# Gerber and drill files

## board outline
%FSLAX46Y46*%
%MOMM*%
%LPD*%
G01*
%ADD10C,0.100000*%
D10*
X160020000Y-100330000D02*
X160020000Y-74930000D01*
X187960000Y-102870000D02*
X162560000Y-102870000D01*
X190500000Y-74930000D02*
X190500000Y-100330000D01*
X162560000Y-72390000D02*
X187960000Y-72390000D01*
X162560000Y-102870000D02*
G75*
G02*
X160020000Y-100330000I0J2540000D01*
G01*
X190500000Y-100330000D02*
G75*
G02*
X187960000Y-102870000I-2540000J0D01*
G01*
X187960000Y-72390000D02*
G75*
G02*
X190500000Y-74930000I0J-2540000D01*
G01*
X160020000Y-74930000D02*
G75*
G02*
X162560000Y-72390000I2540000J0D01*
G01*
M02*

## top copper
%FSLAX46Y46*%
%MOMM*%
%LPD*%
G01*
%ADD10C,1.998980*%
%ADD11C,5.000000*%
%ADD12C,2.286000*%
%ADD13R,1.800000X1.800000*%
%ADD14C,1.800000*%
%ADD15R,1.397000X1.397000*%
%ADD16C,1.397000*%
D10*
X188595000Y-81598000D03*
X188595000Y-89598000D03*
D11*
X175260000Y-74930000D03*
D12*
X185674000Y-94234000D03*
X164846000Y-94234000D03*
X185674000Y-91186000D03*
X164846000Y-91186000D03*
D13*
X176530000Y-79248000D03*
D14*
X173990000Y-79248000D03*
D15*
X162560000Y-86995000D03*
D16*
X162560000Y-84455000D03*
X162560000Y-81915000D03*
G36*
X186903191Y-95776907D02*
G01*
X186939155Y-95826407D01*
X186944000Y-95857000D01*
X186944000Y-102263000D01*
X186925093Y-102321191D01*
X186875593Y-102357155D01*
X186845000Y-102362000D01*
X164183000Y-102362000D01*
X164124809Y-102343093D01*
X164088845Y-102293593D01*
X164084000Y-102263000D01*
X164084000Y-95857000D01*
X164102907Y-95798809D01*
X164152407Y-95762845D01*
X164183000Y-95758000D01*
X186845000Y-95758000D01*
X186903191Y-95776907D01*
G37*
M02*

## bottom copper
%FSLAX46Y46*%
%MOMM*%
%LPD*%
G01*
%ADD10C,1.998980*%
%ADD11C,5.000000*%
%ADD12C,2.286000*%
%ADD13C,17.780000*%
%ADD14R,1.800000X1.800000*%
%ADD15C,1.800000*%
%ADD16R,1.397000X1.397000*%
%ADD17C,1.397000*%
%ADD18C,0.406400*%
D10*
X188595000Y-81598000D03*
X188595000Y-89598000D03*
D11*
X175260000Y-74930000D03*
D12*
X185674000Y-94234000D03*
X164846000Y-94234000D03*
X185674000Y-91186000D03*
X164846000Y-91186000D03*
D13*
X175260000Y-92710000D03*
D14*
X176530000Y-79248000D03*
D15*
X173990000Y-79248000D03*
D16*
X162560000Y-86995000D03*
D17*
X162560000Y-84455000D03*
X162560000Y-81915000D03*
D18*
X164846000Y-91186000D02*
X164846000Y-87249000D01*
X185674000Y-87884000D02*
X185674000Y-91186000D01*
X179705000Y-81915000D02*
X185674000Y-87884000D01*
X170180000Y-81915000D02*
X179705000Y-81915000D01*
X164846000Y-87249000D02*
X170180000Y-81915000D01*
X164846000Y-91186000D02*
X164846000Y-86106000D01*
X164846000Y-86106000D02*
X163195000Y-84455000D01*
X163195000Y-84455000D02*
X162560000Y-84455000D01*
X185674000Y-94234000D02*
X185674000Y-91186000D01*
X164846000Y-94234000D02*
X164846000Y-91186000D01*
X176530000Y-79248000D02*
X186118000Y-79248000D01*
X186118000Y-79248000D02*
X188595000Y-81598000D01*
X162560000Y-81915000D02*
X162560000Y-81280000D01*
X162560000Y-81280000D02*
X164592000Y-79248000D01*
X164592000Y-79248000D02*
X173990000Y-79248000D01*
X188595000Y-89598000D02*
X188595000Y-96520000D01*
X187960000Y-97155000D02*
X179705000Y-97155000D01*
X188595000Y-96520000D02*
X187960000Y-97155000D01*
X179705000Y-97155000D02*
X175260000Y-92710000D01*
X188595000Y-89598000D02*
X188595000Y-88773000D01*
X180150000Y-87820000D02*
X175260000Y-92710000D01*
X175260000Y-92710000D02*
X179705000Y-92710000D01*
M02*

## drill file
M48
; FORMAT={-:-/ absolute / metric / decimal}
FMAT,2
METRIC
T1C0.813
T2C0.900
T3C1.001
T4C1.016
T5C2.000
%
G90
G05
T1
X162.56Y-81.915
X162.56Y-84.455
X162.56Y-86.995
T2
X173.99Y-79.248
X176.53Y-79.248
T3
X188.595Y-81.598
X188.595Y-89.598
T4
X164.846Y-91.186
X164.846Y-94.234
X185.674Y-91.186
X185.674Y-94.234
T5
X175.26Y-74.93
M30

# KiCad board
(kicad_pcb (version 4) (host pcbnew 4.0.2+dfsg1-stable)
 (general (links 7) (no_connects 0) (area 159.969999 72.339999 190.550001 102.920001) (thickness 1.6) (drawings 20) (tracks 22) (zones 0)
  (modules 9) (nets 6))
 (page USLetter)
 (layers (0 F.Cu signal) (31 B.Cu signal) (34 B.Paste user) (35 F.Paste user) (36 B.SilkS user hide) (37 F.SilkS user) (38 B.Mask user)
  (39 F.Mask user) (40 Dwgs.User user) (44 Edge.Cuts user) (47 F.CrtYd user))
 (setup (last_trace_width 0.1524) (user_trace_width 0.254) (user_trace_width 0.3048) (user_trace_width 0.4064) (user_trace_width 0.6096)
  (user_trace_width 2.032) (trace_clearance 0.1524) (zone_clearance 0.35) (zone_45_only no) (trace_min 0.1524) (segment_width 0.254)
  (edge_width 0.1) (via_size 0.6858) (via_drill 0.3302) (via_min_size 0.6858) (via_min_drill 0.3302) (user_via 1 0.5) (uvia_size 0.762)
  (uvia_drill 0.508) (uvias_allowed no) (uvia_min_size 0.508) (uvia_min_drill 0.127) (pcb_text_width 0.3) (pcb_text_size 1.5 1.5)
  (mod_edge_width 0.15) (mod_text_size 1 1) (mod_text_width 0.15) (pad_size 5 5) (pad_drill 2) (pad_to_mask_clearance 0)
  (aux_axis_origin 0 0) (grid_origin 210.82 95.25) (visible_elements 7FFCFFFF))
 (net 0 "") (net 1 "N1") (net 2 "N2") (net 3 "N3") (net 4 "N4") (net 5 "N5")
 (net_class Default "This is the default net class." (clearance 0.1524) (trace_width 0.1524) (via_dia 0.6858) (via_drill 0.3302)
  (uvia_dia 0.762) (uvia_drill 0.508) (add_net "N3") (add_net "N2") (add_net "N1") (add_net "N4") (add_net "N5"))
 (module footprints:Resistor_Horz (layer F.Cu) (at 188.595 85.598 270)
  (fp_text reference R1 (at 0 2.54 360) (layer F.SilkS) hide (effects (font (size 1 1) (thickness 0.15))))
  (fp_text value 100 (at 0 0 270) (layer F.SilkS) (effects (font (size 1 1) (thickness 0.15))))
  (pad 1 thru_hole circle (at -4 0 270) (size 1.99898 1.99898) (drill 1.00076) (layers *.Cu *.SilkS *.Mask) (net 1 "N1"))
  (pad 2 thru_hole circle (at 4 0 270) (size 1.99898 1.99898) (drill 1.00076) (layers *.Cu *.SilkS *.Mask) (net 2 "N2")))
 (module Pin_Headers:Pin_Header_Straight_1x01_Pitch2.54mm (layer F.Cu) (at 175.26 74.93)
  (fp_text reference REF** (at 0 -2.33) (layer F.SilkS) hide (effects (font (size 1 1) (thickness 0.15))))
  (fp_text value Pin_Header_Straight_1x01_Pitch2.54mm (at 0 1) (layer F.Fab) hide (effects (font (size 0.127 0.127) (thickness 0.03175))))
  (pad 1 thru_hole circle (at 0 0) (size 5 5) (drill 2) (layers *.Cu B.Mask)))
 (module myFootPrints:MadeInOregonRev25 (layer F.Cu) (at 167.64 76.454)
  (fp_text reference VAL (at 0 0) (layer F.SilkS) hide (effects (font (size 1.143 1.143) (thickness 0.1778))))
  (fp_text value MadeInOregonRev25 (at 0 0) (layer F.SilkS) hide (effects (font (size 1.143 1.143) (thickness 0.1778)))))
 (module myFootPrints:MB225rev (layer F.Cu) (at 184.15 76.2)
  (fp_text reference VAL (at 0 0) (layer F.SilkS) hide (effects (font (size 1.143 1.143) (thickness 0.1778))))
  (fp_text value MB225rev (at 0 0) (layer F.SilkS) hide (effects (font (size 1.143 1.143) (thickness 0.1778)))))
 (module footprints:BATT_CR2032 (layer B.Cu) (at 175.26 92.71 180)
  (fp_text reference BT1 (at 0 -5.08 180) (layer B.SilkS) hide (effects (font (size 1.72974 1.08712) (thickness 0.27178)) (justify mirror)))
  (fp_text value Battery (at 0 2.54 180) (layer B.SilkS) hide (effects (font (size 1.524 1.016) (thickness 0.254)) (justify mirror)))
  (pad 1 thru_hole circle (at -10.414 -1.524 180) (size 2.286 2.286) (drill 1.016) (layers *.Cu *.Mask B.SilkS) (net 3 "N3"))
  (pad 1 thru_hole circle (at 10.414 -1.524 180) (size 2.286 2.286) (drill 1.016) (layers *.Cu *.Mask B.SilkS) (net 3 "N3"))
  (pad 1 thru_hole circle (at -10.414 1.524 180) (size 2.286 2.286) (drill 1.016) (layers *.Cu *.Mask B.SilkS) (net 3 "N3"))
  (pad 1 thru_hole circle (at 10.414 1.524 180) (size 2.286 2.286) (drill 1.016) (layers *.Cu *.Mask B.SilkS) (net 3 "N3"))
  (pad 2 smd circle (at 0 0 180) (size 17.78 17.78) (layers B.Cu B.Paste B.Mask) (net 2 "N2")))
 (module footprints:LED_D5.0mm (layer F.Cu) (at 176.53 79.248 180)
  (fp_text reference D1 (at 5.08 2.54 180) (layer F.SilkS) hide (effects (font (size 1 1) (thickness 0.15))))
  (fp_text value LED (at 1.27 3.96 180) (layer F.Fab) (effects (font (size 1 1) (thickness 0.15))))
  (pad 1 thru_hole rect (at 0 0 180) (size 1.8 1.8) (drill 0.9) (layers *.Cu *.Mask) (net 1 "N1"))
  (pad 2 thru_hole circle (at 2.54 0 180) (size 1.8 1.8) (drill 0.9) (layers *.Cu *.Mask) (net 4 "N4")))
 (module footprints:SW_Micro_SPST (layer F.Cu) (at 162.56 84.455 90)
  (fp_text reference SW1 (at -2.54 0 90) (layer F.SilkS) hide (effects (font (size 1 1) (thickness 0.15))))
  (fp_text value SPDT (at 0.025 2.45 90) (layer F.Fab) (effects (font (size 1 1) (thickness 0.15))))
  (pad 1 thru_hole rect (at -2.54 0 90) (size 1.397 1.397) (drill 0.8128) (layers *.Cu *.Mask F.SilkS) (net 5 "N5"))
  (pad 2 thru_hole circle (at 0 0 90) (size 1.397 1.397) (drill 0.8128) (layers *.Cu *.Mask F.SilkS) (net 3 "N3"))
  (pad 3 thru_hole circle (at 2.54 0 90) (size 1.397 1.397) (drill 0.8128) (layers *.Cu *.Mask F.SilkS) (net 4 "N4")))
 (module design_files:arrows (layer F.Cu) (at 179.07 77.47)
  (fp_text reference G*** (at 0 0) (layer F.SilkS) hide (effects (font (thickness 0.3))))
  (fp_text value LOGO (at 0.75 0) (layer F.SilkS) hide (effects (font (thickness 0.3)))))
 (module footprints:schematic (layer F.Cu) (at 175.26 87.503)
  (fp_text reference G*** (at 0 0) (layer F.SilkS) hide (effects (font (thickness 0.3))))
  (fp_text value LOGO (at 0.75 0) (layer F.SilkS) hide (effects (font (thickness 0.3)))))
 (gr_line (start 160.02 100.33) (end 160.02 74.93) (angle 90) (layer Edge.Cuts) (width 0.1))
 (gr_line (start 187.96 102.87) (end 162.56 102.87) (angle 90) (layer Edge.Cuts) (width 0.1))
 (gr_line (start 190.5 74.93) (end 190.5 100.33) (angle 90) (layer Edge.Cuts) (width 0.1))
 (gr_line (start 162.56 72.39) (end 187.96 72.39) (angle 90) (layer Edge.Cuts) (width 0.1))
 (gr_arc (start 162.56 100.33) (end 162.56 102.87) (angle 90) (layer Edge.Cuts) (width 0.1))
 (gr_arc (start 187.96 100.33) (end 190.5 100.33) (angle 90) (layer Edge.Cuts) (width 0.1))
 (gr_arc (start 187.96 74.93) (end 187.96 72.39) (angle 90) (layer Edge.Cuts) (width 0.1))
 (gr_arc (start 162.56 74.93) (end 160.02 74.93) (angle 90) (layer Edge.Cuts) (width 0.1))
 (segment (start 164.846 91.186) (end 164.846 87.249) (width 0.4064) (layer B.Cu) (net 3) (status 10))
 (segment (start 185.674 87.884) (end 185.674 91.186) (width 0.4064) (layer B.Cu) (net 3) (status 20))
 (segment (start 179.705 81.915) (end 185.674 87.884) (width 0.4064) (layer B.Cu) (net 3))
 (segment (start 170.18 81.915) (end 179.705 81.915) (width 0.4064) (layer B.Cu) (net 3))
 (segment (start 164.846 87.249) (end 170.18 81.915) (width 0.4064) (layer B.Cu) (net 3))
 (segment (start 164.846 91.186) (end 164.846 86.106) (width 0.4064) (layer B.Cu) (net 3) (status 10))
 (segment (start 164.846 86.106) (end 163.195 84.455) (width 0.4064) (layer B.Cu) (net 3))
 (segment (start 163.195 84.455) (end 162.56 84.455) (width 0.4064) (layer B.Cu) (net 3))
 (segment (start 185.674 94.234) (end 185.674 91.186) (width 0.4064) (layer B.Cu) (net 3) (status 30))
 (segment (start 164.846 94.234) (end 164.846 91.186) (width 0.4064) (layer B.Cu) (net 3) (status 30))
 (segment (start 176.53 79.248) (end 186.118 79.248) (width 0.4064) (layer B.Cu) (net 1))
 (segment (start 186.118 79.248) (end 188.595 81.598) (width 0.4064) (layer B.Cu) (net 1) (status 20))
 (segment (start 162.56 81.915) (end 162.56 81.28) (width 0.4064) (layer B.Cu) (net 4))
 (segment (start 162.56 81.28) (end 164.592 79.248) (width 0.4064) (layer B.Cu) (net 4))
 (segment (start 164.592 79.248) (end 173.99 79.248) (width 0.4064) (layer B.Cu) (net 4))
 (segment (start 188.595 89.598) (end 188.595 96.52) (width 0.4064) (layer B.Cu) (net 2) (status 10))
 (segment (start 187.96 97.155) (end 179.705 97.155) (width 0.4064) (layer B.Cu) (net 2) (status 20))
 (segment (start 188.595 96.52) (end 187.96 97.155) (width 0.4064) (layer B.Cu) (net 2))
 (segment (start 179.705 97.155) (end 175.26 92.71) (width 0.4064) (layer B.Cu) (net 2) (status 30))
 (segment (start 188.595 89.598) (end 188.595 88.773) (width 0.4064) (layer B.Cu) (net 2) (status 30))
 (segment (start 180.15 87.82) (end 175.26 92.71) (width 0.4064) (layer B.Cu) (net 2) (status 30))
 (segment (start 175.26 92.71) (end 179.705 92.71) (width 0.4064) (layer B.Cu) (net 2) (status 30))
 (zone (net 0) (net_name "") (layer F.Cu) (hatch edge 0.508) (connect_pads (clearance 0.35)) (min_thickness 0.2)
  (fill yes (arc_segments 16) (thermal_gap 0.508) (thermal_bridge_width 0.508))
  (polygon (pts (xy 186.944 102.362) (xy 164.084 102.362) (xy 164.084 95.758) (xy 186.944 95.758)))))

